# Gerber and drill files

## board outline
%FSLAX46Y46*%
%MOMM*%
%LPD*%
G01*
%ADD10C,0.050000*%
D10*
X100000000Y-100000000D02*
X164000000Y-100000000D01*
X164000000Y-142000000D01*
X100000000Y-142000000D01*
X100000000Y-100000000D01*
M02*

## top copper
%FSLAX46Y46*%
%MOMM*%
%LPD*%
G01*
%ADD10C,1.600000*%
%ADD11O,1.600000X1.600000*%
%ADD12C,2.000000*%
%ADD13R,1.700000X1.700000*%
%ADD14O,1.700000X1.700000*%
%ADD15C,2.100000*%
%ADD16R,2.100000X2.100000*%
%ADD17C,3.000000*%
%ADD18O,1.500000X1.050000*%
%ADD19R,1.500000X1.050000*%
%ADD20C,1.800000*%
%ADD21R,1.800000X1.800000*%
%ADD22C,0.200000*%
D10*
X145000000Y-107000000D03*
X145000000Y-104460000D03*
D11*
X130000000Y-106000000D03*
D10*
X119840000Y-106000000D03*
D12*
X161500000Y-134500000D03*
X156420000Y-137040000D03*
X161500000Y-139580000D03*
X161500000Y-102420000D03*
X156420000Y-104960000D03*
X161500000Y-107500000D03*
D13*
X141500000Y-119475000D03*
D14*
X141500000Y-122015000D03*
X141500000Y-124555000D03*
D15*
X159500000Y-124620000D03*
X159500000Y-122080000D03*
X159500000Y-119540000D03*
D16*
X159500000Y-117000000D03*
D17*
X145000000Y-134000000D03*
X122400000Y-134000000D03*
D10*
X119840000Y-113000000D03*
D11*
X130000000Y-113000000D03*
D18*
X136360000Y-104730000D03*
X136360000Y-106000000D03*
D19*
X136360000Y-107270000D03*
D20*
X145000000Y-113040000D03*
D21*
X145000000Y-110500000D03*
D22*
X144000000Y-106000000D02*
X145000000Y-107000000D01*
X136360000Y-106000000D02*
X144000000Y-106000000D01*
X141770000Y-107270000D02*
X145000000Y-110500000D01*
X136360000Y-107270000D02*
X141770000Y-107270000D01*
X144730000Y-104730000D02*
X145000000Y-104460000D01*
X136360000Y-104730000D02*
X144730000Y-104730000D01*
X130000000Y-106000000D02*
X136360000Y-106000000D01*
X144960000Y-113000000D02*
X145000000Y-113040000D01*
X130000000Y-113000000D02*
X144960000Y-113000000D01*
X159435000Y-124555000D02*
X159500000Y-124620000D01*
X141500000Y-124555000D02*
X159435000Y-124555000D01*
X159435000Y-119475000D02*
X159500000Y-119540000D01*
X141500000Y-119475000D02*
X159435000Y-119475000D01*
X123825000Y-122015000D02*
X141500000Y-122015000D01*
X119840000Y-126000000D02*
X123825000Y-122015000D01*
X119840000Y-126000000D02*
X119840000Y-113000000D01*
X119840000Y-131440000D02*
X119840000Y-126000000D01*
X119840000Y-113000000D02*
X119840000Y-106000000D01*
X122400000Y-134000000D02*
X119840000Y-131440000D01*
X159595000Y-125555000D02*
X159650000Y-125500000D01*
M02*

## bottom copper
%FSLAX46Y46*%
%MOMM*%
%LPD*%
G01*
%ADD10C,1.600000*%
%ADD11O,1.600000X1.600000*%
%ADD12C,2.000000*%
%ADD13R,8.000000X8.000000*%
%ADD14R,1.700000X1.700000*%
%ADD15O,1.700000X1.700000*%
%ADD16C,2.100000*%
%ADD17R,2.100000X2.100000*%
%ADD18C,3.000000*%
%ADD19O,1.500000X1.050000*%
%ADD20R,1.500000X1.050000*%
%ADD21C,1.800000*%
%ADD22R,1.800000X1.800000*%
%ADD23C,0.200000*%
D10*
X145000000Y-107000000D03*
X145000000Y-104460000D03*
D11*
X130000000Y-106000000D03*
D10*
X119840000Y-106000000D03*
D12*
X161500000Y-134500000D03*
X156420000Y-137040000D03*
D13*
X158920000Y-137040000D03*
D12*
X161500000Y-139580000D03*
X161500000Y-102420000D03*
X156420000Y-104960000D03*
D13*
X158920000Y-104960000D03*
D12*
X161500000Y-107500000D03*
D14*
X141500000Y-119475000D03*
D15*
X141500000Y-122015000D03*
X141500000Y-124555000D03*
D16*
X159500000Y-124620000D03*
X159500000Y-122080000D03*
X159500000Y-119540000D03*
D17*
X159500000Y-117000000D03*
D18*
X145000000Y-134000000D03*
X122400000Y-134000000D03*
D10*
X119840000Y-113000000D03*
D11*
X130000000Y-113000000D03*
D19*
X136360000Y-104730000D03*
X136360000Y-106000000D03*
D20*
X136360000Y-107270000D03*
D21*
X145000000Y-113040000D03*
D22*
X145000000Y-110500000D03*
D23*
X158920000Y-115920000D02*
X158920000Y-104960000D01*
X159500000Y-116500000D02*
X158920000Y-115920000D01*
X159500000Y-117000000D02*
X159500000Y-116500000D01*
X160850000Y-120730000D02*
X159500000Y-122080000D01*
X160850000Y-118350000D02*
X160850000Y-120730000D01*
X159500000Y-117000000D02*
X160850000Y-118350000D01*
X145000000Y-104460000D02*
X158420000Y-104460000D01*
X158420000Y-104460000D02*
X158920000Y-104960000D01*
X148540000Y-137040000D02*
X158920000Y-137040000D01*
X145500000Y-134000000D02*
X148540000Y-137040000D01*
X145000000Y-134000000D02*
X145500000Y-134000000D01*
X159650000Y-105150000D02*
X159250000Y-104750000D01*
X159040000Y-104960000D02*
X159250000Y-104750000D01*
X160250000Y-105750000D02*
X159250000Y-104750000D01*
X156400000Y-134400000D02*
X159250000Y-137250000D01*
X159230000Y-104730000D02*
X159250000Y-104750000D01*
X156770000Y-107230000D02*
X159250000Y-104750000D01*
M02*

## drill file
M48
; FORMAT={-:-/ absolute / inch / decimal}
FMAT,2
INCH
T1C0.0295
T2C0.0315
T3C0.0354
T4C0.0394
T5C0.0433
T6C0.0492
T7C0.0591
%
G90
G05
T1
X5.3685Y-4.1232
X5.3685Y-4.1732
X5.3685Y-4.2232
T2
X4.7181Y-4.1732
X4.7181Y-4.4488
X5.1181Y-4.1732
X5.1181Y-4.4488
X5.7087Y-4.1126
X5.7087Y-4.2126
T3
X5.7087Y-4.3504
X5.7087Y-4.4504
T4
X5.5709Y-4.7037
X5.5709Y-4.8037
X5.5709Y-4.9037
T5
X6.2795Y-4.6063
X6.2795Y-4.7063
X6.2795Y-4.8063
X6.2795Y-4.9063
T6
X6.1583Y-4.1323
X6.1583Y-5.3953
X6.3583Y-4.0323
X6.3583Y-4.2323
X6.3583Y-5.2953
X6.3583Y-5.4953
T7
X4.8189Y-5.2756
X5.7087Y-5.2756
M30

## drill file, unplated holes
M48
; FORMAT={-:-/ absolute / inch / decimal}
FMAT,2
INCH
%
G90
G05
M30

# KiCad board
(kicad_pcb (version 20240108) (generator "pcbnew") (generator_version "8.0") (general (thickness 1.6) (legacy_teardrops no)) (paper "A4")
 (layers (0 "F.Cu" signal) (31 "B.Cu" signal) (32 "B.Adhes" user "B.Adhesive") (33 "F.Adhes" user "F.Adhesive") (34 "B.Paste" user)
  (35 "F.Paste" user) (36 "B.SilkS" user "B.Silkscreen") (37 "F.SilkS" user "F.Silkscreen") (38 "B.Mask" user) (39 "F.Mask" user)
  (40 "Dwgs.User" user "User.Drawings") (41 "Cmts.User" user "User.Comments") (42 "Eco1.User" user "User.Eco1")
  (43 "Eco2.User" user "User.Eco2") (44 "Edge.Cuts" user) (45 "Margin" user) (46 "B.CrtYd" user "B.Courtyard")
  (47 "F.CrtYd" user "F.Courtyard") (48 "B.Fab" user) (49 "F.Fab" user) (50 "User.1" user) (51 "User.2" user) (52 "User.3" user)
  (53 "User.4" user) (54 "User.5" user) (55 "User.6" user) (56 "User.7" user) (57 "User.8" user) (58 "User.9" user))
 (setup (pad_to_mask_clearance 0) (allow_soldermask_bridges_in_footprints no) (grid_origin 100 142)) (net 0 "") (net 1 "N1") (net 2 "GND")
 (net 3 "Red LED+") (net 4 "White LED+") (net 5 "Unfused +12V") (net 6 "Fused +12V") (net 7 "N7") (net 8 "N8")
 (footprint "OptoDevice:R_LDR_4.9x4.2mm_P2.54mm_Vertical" (layer "F.Cu") (at 145 107 90)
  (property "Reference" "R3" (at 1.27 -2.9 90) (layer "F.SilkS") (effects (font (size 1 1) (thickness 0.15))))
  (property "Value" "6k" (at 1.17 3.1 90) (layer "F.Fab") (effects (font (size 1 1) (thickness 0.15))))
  (pad "1" thru_hole circle (at 0 0 90) (size 1.6 1.6) (drill 0.8) (layers "*.Cu" "*.Mask") (remove_unused_layers no) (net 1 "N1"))
  (pad "2" thru_hole circle (at 2.54 0 90) (size 1.6 1.6) (drill 0.8) (layers "*.Cu" "*.Mask") (remove_unused_layers no) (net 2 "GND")))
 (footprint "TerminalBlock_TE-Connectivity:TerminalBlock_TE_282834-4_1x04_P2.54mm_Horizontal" (layer "F.Cu") (at 159.5 117 -90)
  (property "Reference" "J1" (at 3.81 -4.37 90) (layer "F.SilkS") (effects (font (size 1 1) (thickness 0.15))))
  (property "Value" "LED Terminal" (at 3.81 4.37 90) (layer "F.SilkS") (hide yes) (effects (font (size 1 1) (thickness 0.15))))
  (pad "1" thru_hole rect (at 0 0 270) (size 2.1 2.1) (drill 1.1) (layers "*.Cu" "*.Mask") (remove_unused_layers no) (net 2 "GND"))
  (pad "2" thru_hole circle (at 2.54 0 270) (size 2.1 2.1) (drill 1.1) (layers "*.Cu" "*.Mask") (remove_unused_layers no) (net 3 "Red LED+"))
  (pad "3" thru_hole circle (at 5.08 0 270) (size 2.1 2.1) (drill 1.1) (layers "*.Cu" "*.Mask") (remove_unused_layers no) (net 2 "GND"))
  (pad "4" thru_hole circle (at 7.62 0 270) (size 2.1 2.1) (drill 1.1) (layers "*.Cu" "*.Mask") (remove_unused_layers no)
   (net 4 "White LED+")))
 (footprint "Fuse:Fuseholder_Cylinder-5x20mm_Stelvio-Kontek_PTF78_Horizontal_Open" (layer "F.Cu") (at 145 134 180)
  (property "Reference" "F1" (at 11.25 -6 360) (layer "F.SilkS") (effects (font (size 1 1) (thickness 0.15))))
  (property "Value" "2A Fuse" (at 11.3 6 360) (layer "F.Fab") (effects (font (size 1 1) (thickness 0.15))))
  (pad "1" thru_hole circle (at 0 0 180) (size 3 3) (drill 1.5) (layers "*.Cu" "*.Mask") (remove_unused_layers no) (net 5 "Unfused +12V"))
  (pad "2" thru_hole circle (at 22.6 0 180) (size 3 3) (drill 1.5) (layers "*.Cu" "*.Mask") (remove_unused_layers no) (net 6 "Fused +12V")))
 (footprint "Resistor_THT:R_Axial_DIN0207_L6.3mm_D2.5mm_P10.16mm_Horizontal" (layer "F.Cu") (at 119.84 113)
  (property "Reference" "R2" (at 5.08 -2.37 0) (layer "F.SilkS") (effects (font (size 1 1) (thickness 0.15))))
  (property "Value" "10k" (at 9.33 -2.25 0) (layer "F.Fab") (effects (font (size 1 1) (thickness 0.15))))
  (pad "1" thru_hole circle (at 0 0) (size 1.6 1.6) (drill 0.8) (layers "*.Cu" "*.Mask") (remove_unused_layers no) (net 6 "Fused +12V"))
  (pad "2" thru_hole oval (at 10.16 0) (size 1.6 1.6) (drill 0.8) (layers "*.Cu" "*.Mask") (remove_unused_layers no) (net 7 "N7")))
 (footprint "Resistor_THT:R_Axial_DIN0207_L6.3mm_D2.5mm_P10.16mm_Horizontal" (layer "F.Cu") (at 119.84 106)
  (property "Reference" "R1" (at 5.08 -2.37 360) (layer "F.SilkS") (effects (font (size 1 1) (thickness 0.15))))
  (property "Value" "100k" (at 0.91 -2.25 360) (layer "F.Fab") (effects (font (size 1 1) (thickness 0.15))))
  (pad "1" thru_hole circle (at 0 0) (size 1.6 1.6) (drill 0.8) (layers "*.Cu" "*.Mask") (remove_unused_layers no) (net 6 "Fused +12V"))
  (pad "2" thru_hole oval (at 10.16 0) (size 1.6 1.6) (drill 0.8) (layers "*.Cu" "*.Mask") (remove_unused_layers no) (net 1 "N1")))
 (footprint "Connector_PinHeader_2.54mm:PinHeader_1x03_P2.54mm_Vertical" (layer "F.Cu") (at 141.5 119.475)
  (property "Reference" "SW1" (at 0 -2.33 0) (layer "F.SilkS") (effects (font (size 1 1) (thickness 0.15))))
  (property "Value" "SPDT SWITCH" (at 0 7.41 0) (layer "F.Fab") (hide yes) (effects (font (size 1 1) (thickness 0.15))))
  (pad "1" thru_hole rect (at 0 0) (size 1.7 1.7) (drill 1) (layers "*.Cu" "*.Mask") (remove_unused_layers no) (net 3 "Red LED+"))
  (pad "2" thru_hole oval (at 0 2.54) (size 1.7 1.7) (drill 1) (layers "*.Cu" "*.Mask") (remove_unused_layers no) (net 6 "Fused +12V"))
  (pad "3" thru_hole oval (at 0 5.08) (size 1.7 1.7) (drill 1) (layers "*.Cu" "*.Mask") (remove_unused_layers no) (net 4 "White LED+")))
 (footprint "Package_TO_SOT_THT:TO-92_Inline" (layer "F.Cu") (at 136.36 107.27 90)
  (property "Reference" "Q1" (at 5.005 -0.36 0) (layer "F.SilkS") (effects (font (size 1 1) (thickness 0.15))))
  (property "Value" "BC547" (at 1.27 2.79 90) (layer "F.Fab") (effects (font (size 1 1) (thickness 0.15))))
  (pad "1" thru_hole rect (at 0 0 90) (size 1.05 1.5) (drill 0.75) (layers "*.Cu" "*.Mask") (remove_unused_layers no) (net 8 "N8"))
  (pad "2" thru_hole oval (at 1.27 0 90) (size 1.05 1.5) (drill 0.75) (layers "*.Cu" "*.Mask") (remove_unused_layers no) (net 1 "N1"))
  (pad "3" thru_hole oval (at 2.54 0 90) (size 1.05 1.5) (drill 0.75) (layers "*.Cu" "*.Mask") (remove_unused_layers no) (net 2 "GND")))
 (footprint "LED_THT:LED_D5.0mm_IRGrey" (layer "F.Cu") (at 145 110.5 -90)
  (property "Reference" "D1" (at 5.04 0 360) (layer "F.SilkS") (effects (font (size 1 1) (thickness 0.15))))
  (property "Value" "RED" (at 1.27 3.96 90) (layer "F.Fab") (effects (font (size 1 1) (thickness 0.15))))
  (pad "1" thru_hole rect (at 0 0 270) (size 1.8 1.8) (drill 0.9) (layers "*.Cu" "*.Mask") (remove_unused_layers no) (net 8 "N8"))
  (pad "2" thru_hole circle (at 2.54 0 270) (size 1.8 1.8) (drill 0.9) (layers "*.Cu" "*.Mask") (remove_unused_layers no) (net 7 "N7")))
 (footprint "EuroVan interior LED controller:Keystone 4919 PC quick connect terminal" (layer "B.Cu") (at 156.42 104.96 -90)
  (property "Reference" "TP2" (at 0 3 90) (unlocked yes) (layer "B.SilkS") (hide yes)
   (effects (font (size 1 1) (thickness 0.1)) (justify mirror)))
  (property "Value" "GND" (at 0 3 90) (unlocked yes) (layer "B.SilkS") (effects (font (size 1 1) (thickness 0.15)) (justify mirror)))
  (pad "1" thru_hole circle (at -2.54 -5.08 270) (size 2 2) (drill 1.25) (layers "*.Cu" "*.Mask") (remove_unused_layers no) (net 2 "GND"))
  (pad "1" smd rect (at 0 -2.5 270) (size 8 8) (layers "B.Cu" "B.Mask") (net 2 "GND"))
  (pad "1" thru_hole circle (at 0 0 270) (size 2 2) (drill 1.25) (layers "*.Cu" "*.Mask") (remove_unused_layers no) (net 2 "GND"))
  (pad "1" thru_hole circle (at 2.54 -5.08 270) (size 2 2) (drill 1.25) (layers "*.Cu" "*.Mask") (remove_unused_layers no) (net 2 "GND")))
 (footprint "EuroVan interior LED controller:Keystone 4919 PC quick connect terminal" (layer "B.Cu") (at 156.42 137.04 -90)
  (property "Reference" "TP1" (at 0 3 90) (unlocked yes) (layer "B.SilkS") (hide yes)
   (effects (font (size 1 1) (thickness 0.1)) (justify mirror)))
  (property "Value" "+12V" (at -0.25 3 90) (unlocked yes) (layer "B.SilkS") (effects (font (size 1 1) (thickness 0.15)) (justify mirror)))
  (pad "1" thru_hole circle (at -2.54 -5.08 270) (size 2 2) (drill 1.25) (layers "*.Cu" "*.Mask") (remove_unused_layers no)
   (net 5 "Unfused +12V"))
  (pad "1" smd rect (at 0 -2.5 270) (size 8 8) (layers "B.Cu" "B.Mask") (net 5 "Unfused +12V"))
  (pad "1" thru_hole circle (at 0 0 270) (size 2 2) (drill 1.25) (layers "*.Cu" "*.Mask") (remove_unused_layers no) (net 5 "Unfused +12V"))
  (pad "1" thru_hole circle (at 2.54 -5.08 270) (size 2 2) (drill 1.25) (layers "*.Cu" "*.Mask") (remove_unused_layers no)
   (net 5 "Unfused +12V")))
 (gr_rect (start 100 100) (end 164 142) (stroke (width 0.05) (type default)) (fill none) (layer "Edge.Cuts"))
 (segment (start 144.96 113) (end 145 113.04) (width 0.2) (layer "F.Cu") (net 7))
 (segment (start 130 113) (end 144.96 113) (width 0.2) (layer "F.Cu") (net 7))
 (segment (start 136.36 107.27) (end 141.77 107.27) (width 0.2) (layer "F.Cu") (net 8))
 (segment (start 141.77 107.27) (end 145 110.5) (width 0.2) (layer "F.Cu") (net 8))
 (segment (start 130 106) (end 136.36 106) (width 0.2) (layer "F.Cu") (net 1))
 (segment (start 144 106) (end 145 107) (width 0.2) (layer "F.Cu") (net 1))
 (segment (start 136.36 106) (end 144 106) (width 0.2) (layer "F.Cu") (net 1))
 (segment (start 136.36 104.73) (end 144.73 104.73) (width 0.2) (layer "F.Cu") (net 2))
 (segment (start 144.73 104.73) (end 145 104.46) (width 0.2) (layer "F.Cu") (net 2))
 (segment (start 160.85 120.73) (end 159.5 122.08) (width 0.2) (layer "B.Cu") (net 2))
 (segment (start 159.5 117) (end 159.5 116.5) (width 0.2) (layer "B.Cu") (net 2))
 (segment (start 159.04 104.96) (end 159.25 104.75) (width 0.2) (layer "B.Cu") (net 2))
 (segment (start 159.5 116.5) (end 158.92 115.92) (width 0.2) (layer "B.Cu") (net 2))
 (segment (start 158.42 104.46) (end 158.92 104.96) (width 0.2) (layer "B.Cu") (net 2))
 (segment (start 158.92 115.92) (end 158.92 104.96) (width 0.2) (layer "B.Cu") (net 2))
 (segment (start 159.23 104.73) (end 159.25 104.75) (width 0.2) (layer "B.Cu") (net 2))
 (segment (start 160.85 118.35) (end 160.85 120.73) (width 0.2) (layer "B.Cu") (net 2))
 (segment (start 159.65 105.15) (end 159.25 104.75) (width 0.2) (layer "B.Cu") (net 2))
 (segment (start 156.77 107.23) (end 159.25 104.75) (width 0.2) (layer "B.Cu") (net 2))
 (segment (start 159.5 117) (end 160.85 118.35) (width 0.2) (layer "B.Cu") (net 2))
 (segment (start 160.25 105.75) (end 159.25 104.75) (width 0.2) (layer "B.Cu") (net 2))
 (segment (start 145 104.46) (end 158.42 104.46) (width 0.2) (layer "B.Cu") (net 2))
 (segment (start 119.84 126) (end 119.84 113) (width 0.2) (layer "F.Cu") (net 6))
 (segment (start 123.825 122.015) (end 141.5 122.015) (width 0.2) (layer "F.Cu") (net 6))
 (segment (start 122.4 134) (end 119.84 131.44) (width 0.2) (layer "F.Cu") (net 6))
 (segment (start 119.84 126) (end 123.825 122.015) (width 0.2) (layer "F.Cu") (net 6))
 (segment (start 119.84 131.44) (end 119.84 126) (width 0.2) (layer "F.Cu") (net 6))
 (segment (start 119.84 113) (end 119.84 106) (width 0.2) (layer "F.Cu") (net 6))
 (segment (start 159.435 124.555) (end 159.5 124.62) (width 0.2) (layer "F.Cu") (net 4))
 (segment (start 159.595 125.555) (end 159.65 125.5) (width 0.2) (layer "F.Cu") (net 4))
 (segment (start 141.5 124.555) (end 159.435 124.555) (width 0.2) (layer "F.Cu") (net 4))
 (segment (start 141.5 119.475) (end 159.435 119.475) (width 0.2) (layer "F.Cu") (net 3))
 (segment (start 159.435 119.475) (end 159.5 119.54) (width 0.2) (layer "F.Cu") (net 3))
 (segment (start 156.4 134.4) (end 159.25 137.25) (width 0.2) (layer "B.Cu") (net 5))
 (segment (start 145 134) (end 145.5 134) (width 0.2) (layer "B.Cu") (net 5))
 (segment (start 148.54 137.04) (end 158.92 137.04) (width 0.2) (layer "B.Cu") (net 5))
 (segment (start 145.5 134) (end 148.54 137.04) (width 0.2) (layer "B.Cu") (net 5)))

